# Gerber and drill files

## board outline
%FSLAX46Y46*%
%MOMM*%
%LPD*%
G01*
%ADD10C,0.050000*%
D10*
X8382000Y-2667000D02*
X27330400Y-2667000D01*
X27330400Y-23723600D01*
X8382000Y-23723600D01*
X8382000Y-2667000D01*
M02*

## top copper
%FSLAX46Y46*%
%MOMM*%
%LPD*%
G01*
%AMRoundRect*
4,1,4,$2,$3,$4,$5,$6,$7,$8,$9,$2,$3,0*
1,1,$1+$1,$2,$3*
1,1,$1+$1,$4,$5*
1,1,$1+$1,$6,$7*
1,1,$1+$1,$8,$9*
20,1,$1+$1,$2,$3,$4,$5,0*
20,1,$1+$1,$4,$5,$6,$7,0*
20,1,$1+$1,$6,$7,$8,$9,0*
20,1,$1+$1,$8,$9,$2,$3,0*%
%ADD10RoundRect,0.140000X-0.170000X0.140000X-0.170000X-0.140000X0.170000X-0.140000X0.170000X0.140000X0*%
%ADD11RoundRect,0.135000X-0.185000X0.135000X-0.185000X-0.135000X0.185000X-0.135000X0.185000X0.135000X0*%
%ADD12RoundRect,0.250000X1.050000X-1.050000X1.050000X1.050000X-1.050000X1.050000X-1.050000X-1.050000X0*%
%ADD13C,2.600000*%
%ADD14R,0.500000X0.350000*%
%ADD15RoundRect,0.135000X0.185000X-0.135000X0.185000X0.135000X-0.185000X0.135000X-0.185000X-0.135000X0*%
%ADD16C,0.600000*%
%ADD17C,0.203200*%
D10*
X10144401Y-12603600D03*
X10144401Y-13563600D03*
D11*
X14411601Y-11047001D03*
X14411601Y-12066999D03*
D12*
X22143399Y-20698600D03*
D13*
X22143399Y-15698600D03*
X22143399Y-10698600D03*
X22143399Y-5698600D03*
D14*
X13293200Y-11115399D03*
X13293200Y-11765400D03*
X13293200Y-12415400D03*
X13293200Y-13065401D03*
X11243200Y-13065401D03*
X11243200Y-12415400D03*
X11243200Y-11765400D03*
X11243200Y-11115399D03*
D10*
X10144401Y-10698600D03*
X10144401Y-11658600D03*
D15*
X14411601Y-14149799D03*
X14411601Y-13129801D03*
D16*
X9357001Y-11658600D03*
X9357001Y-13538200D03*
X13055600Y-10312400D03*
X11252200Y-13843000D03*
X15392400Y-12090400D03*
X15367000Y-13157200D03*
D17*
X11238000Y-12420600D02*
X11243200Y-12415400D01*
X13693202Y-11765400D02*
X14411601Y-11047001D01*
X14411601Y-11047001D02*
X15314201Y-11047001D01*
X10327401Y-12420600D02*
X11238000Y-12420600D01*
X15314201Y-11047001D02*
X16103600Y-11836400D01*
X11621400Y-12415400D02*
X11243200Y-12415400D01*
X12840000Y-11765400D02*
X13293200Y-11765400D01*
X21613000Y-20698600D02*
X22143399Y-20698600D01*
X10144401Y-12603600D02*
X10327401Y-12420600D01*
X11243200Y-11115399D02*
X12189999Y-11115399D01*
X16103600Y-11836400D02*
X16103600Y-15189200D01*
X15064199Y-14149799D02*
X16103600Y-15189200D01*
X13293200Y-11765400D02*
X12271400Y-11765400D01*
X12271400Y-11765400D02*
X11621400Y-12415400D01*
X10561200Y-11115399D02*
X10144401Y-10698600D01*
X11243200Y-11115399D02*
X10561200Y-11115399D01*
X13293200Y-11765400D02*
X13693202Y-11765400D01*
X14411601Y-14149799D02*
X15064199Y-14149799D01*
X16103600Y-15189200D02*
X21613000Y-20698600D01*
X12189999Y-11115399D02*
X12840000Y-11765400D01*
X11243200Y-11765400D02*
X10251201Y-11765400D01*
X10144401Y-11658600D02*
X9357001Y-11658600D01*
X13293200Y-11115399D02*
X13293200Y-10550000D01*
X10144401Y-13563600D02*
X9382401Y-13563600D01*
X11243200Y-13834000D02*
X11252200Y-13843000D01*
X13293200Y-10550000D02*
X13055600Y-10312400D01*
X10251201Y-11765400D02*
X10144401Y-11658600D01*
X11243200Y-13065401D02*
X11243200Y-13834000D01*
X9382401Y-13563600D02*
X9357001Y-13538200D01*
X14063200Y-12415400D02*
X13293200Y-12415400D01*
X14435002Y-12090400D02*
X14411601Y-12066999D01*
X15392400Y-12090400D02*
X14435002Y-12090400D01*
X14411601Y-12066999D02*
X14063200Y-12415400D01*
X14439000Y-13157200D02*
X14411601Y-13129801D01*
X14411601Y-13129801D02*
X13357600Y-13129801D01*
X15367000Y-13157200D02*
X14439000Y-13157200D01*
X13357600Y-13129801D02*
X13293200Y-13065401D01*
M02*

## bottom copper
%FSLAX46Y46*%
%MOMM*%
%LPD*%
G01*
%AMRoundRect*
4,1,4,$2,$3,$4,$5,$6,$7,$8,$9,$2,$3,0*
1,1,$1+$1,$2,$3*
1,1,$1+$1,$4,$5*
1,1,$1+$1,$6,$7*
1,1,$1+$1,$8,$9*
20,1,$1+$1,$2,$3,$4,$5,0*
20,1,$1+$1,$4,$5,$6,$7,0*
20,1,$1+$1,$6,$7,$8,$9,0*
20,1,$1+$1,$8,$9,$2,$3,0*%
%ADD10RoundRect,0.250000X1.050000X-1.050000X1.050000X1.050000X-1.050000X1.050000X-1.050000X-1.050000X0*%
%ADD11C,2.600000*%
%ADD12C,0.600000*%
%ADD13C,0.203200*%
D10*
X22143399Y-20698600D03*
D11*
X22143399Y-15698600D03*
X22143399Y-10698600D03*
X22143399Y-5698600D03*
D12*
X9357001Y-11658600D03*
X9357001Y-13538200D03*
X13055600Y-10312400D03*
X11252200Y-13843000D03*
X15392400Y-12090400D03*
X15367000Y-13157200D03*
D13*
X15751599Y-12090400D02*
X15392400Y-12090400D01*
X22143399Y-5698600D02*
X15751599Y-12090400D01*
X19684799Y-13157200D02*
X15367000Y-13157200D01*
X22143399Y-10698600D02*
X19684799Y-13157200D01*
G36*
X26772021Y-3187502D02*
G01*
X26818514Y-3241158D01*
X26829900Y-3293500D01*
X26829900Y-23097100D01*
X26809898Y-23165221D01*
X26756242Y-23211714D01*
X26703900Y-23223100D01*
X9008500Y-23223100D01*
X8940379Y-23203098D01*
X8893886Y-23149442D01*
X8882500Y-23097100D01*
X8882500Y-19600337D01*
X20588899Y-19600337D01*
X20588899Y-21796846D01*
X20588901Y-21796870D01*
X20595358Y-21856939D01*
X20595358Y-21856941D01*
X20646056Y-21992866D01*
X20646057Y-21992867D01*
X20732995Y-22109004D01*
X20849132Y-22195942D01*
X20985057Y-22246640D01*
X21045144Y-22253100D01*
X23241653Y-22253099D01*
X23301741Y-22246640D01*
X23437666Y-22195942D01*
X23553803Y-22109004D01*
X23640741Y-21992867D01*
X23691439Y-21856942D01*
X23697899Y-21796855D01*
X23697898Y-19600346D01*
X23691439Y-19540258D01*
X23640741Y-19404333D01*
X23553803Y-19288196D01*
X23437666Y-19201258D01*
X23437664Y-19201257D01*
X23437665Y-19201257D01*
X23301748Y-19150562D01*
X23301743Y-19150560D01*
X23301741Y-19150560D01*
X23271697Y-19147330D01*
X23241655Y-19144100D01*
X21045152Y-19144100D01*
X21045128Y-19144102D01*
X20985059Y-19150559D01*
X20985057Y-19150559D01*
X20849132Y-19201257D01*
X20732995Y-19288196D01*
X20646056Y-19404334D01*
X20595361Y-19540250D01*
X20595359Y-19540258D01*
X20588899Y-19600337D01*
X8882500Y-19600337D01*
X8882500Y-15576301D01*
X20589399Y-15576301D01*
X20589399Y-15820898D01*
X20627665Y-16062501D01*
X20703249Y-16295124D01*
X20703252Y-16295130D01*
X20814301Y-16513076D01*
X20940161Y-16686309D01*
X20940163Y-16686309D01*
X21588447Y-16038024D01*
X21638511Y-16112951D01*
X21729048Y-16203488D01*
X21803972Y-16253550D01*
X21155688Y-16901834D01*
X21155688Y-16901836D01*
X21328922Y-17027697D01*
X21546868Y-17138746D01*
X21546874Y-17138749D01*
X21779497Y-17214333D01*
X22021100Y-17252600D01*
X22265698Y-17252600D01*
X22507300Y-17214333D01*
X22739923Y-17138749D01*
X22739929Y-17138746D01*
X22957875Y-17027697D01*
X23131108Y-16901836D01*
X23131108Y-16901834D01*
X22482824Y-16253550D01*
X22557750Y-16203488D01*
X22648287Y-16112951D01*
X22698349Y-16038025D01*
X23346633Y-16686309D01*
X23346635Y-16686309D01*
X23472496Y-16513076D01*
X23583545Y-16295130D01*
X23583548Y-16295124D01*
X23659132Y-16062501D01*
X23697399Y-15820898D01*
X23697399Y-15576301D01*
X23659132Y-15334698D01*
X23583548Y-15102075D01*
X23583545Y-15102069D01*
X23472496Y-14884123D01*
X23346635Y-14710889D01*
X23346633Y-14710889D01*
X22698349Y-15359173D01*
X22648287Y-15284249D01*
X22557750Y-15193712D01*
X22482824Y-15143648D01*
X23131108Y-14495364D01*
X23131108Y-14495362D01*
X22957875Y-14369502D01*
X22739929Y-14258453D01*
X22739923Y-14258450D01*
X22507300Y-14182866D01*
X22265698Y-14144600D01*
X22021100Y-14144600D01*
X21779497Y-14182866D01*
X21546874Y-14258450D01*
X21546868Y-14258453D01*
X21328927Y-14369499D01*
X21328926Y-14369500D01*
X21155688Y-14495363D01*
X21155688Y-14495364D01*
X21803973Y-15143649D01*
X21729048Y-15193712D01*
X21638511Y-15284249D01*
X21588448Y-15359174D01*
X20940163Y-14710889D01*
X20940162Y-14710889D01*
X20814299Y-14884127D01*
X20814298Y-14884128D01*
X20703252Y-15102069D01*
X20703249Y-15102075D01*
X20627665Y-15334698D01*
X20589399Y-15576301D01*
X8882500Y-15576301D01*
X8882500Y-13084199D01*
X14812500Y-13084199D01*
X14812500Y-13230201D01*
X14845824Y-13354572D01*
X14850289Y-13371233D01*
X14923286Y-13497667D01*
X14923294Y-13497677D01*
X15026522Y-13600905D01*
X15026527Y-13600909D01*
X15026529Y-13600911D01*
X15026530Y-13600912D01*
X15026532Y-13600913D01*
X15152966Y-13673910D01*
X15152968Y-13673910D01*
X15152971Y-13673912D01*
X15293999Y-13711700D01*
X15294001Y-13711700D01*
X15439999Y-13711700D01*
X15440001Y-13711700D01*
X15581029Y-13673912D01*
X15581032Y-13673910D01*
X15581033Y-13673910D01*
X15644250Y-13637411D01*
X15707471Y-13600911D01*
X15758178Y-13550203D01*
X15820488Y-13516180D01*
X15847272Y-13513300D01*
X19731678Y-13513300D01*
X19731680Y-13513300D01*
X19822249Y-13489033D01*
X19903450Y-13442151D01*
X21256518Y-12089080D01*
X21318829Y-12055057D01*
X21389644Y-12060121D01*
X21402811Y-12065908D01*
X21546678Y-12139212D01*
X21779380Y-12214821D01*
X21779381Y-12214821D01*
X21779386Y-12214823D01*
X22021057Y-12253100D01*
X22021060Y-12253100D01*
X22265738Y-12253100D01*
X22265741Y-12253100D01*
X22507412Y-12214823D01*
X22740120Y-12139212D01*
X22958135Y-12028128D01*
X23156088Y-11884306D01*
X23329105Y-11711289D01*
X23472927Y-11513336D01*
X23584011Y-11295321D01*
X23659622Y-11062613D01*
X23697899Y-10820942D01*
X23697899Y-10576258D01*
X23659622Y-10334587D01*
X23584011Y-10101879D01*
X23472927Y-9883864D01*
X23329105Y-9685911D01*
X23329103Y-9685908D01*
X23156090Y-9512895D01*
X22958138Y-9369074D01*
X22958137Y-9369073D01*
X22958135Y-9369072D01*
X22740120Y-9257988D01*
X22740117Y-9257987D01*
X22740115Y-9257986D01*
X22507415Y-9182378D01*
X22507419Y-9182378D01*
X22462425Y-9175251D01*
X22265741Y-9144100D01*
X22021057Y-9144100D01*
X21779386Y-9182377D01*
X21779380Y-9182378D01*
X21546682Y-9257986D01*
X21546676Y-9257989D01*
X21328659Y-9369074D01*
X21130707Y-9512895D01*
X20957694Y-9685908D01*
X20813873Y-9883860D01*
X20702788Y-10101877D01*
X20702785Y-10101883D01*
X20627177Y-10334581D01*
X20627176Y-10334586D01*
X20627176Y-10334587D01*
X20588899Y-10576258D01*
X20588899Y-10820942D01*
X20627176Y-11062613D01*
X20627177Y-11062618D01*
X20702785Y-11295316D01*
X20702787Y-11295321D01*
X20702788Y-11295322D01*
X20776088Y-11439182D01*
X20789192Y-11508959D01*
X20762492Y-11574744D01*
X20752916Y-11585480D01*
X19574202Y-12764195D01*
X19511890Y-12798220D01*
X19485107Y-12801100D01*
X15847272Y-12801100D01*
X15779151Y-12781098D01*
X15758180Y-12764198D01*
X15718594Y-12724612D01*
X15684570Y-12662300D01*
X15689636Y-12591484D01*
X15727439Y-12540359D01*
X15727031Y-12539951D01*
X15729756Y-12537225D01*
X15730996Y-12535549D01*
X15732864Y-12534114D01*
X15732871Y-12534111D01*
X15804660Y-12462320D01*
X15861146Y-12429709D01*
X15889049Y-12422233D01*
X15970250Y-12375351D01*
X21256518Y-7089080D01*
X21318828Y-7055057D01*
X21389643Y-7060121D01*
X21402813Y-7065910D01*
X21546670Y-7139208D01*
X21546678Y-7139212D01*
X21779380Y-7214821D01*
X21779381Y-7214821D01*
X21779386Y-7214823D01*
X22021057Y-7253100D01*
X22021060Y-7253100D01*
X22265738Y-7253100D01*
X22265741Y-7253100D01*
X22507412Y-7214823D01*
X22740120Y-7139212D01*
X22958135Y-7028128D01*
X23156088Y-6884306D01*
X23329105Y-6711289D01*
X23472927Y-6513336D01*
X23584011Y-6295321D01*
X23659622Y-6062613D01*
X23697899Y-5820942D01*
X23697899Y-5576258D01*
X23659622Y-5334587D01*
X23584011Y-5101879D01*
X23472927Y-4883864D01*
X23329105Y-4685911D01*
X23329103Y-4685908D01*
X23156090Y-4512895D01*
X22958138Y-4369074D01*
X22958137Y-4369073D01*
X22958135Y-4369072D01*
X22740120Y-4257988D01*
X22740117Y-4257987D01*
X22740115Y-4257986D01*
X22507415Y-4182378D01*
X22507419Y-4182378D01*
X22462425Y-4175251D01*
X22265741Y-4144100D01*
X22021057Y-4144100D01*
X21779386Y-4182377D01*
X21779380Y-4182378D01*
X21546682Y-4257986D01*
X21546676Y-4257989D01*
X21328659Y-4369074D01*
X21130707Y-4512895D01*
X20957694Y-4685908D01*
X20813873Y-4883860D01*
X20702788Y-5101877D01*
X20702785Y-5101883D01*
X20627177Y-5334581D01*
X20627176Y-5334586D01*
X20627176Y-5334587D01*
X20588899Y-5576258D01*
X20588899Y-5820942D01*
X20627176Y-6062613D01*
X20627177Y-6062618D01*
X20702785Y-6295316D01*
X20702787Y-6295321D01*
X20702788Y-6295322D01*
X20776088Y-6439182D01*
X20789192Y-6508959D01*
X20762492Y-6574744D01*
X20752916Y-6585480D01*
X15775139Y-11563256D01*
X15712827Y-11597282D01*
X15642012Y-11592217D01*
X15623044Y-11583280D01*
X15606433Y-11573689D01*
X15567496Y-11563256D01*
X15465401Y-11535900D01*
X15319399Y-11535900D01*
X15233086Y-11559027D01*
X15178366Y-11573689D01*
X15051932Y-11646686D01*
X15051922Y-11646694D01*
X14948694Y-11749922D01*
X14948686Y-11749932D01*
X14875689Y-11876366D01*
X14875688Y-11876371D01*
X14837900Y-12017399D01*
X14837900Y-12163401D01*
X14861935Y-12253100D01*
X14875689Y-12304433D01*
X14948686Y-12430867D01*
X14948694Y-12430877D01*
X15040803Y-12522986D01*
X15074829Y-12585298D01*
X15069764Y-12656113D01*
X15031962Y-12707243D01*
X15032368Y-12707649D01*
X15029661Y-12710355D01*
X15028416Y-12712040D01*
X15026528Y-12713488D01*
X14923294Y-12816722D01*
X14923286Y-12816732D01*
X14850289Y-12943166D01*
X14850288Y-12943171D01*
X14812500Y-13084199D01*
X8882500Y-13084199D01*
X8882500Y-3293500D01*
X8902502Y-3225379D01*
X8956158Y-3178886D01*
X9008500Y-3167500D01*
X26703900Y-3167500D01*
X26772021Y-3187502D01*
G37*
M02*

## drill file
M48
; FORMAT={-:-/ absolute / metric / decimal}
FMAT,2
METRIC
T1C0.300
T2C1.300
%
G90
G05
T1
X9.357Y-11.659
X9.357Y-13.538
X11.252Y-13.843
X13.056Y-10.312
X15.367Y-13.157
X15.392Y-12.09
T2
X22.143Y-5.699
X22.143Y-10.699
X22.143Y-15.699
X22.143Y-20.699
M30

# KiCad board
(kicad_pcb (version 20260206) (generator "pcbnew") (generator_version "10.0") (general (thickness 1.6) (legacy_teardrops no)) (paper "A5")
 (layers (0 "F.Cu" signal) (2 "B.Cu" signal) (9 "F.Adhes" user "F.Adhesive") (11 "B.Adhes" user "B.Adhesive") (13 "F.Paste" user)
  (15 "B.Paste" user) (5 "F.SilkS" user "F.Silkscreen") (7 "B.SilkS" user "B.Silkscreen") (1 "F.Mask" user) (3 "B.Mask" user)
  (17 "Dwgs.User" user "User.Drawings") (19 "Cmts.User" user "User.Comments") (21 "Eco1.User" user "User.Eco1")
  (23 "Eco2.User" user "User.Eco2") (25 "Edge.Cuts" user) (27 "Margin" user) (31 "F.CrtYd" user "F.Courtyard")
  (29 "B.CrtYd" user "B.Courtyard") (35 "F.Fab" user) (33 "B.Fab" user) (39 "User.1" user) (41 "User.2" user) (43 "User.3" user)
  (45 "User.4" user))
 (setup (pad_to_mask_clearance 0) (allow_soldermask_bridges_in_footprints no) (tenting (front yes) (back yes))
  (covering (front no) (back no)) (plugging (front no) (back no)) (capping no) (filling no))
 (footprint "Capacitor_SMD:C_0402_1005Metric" (layer "F.Cu") (at 10.144401 13.0836 -90)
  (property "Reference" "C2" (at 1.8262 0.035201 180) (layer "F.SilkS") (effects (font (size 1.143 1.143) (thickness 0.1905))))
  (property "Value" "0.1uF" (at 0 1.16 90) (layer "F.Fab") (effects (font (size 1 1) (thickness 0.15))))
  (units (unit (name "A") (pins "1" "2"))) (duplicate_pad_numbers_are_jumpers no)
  (pad "1" smd roundrect (at -0.48 0 270) (size 0.56 0.62) (layers "F.Cu" "F.Mask" "F.Paste") (roundrect_rratio 0.25) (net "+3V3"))
  (pad "2" smd roundrect (at 0.48 0 270) (size 0.56 0.62) (layers "F.Cu" "F.Mask" "F.Paste") (roundrect_rratio 0.25) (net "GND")))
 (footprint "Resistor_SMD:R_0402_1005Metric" (layer "F.Cu") (at 14.411601 11.557 -90)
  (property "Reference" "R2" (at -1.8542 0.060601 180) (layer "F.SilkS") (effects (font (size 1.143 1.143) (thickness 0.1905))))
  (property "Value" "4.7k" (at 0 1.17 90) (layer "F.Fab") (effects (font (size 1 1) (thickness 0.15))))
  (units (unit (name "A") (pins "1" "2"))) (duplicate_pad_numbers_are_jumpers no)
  (pad "1" smd roundrect (at -0.509999 0 270) (size 0.54 0.64) (layers "F.Cu" "F.Mask" "F.Paste") (roundrect_rratio 0.25) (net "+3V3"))
  (pad "2" smd roundrect (at 0.509999 0 270) (size 0.54 0.64) (layers "F.Cu" "F.Mask" "F.Paste") (roundrect_rratio 0.25) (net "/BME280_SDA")))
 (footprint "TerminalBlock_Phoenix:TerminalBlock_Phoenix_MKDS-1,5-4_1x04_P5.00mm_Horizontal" (layer "F.Cu") (at 22.143399 20.6986 90)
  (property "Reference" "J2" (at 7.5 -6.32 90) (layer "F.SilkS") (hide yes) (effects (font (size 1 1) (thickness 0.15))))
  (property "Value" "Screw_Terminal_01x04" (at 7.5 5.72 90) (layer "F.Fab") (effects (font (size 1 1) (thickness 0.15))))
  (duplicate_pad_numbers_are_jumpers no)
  (pad "1" thru_hole roundrect (at 0 0 90) (size 2.6 2.6) (drill 1.3) (layers "*.Cu" "*.Mask") (remove_unused_layers no)
   (roundrect_rratio 0.096154) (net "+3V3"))
  (pad "2" thru_hole circle (at 5 0 90) (size 2.6 2.6) (drill 1.3) (layers "*.Cu" "*.Mask") (remove_unused_layers no) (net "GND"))
  (pad "3" thru_hole circle (at 10 0 90) (size 2.6 2.6) (drill 1.3) (layers "*.Cu" "*.Mask") (remove_unused_layers no) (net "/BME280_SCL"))
  (pad "4" thru_hole circle (at 15 0 90) (size 2.6 2.6) (drill 1.3) (layers "*.Cu" "*.Mask") (remove_unused_layers no) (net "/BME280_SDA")))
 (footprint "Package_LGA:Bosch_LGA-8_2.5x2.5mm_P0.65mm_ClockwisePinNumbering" (layer "F.Cu") (at 12.2682 12.0904 -90)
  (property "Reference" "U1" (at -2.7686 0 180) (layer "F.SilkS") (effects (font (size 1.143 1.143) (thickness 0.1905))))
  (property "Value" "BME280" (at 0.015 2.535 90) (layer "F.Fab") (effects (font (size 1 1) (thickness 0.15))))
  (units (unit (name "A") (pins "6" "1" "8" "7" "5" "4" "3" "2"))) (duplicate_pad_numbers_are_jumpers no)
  (pad "1" smd rect (at -0.975001 -1.025) (size 0.5 0.35) (layers "F.Cu" "F.Mask" "F.Paste") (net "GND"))
  (pad "2" smd rect (at -0.325 -1.025) (size 0.5 0.35) (layers "F.Cu" "F.Mask" "F.Paste") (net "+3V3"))
  (pad "3" smd rect (at 0.325 -1.025) (size 0.5 0.35) (layers "F.Cu" "F.Mask" "F.Paste") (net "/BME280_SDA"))
  (pad "4" smd rect (at 0.975001 -1.025) (size 0.5 0.35) (layers "F.Cu" "F.Mask" "F.Paste") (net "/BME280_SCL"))
  (pad "5" smd rect (at 0.975001 1.025) (size 0.5 0.35) (layers "F.Cu" "F.Mask" "F.Paste") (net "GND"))
  (pad "6" smd rect (at 0.325 1.025) (size 0.5 0.35) (layers "F.Cu" "F.Mask" "F.Paste") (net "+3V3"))
  (pad "7" smd rect (at -0.325 1.025) (size 0.5 0.35) (layers "F.Cu" "F.Mask" "F.Paste") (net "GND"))
  (pad "8" smd rect (at -0.975001 1.025) (size 0.5 0.35) (layers "F.Cu" "F.Mask" "F.Paste") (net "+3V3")))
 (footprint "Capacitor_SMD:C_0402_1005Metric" (layer "F.Cu") (at 10.144401 11.1786 -90)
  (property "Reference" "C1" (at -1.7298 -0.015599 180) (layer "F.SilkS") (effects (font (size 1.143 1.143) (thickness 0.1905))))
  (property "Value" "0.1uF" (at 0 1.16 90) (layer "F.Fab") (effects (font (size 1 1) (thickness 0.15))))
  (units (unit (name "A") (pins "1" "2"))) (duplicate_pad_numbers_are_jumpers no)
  (pad "1" smd roundrect (at -0.48 0 270) (size 0.56 0.62) (layers "F.Cu" "F.Mask" "F.Paste") (roundrect_rratio 0.25) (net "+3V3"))
  (pad "2" smd roundrect (at 0.48 0 270) (size 0.56 0.62) (layers "F.Cu" "F.Mask" "F.Paste") (roundrect_rratio 0.25) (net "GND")))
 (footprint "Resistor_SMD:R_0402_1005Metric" (layer "F.Cu") (at 14.411601 13.6398 90)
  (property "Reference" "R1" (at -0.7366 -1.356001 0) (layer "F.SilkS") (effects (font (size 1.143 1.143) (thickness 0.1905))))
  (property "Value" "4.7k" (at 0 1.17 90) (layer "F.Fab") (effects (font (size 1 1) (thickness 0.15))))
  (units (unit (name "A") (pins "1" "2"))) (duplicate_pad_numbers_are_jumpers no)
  (pad "1" smd roundrect (at -0.509999 0 90) (size 0.54 0.64) (layers "F.Cu" "F.Mask" "F.Paste") (roundrect_rratio 0.25) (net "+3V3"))
  (pad "2" smd roundrect (at 0.509999 0 90) (size 0.54 0.64) (layers "F.Cu" "F.Mask" "F.Paste") (roundrect_rratio 0.25) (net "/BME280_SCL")))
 (gr_rect (start 8.382 2.667) (end 27.3304 23.7236) (stroke (width 0.05) (type default)) (fill no) (layer "Edge.Cuts"))
 (segment (start 11.238 12.4206) (end 11.2432 12.4154) (width 0.2032) (layer "F.Cu") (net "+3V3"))
 (segment (start 13.693202 11.7654) (end 14.411601 11.047001) (width 0.2032) (layer "F.Cu") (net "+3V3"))
 (segment (start 14.411601 11.047001) (end 15.314201 11.047001) (width 0.2032) (layer "F.Cu") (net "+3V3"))
 (segment (start 10.327401 12.4206) (end 11.238 12.4206) (width 0.2032) (layer "F.Cu") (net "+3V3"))
 (segment (start 15.314201 11.047001) (end 16.1036 11.8364) (width 0.2032) (layer "F.Cu") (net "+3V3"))
 (segment (start 11.6214 12.4154) (end 11.2432 12.4154) (width 0.2032) (layer "F.Cu") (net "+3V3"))
 (segment (start 12.84 11.7654) (end 13.2932 11.7654) (width 0.2032) (layer "F.Cu") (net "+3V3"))
 (segment (start 21.613 20.6986) (end 22.143399 20.6986) (width 0.2032) (layer "F.Cu") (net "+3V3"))
 (segment (start 10.144401 12.6036) (end 10.327401 12.4206) (width 0.2032) (layer "F.Cu") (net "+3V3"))
 (segment (start 11.2432 11.115399) (end 12.189999 11.115399) (width 0.2032) (layer "F.Cu") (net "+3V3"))
 (segment (start 16.1036 11.8364) (end 16.1036 15.1892) (width 0.2032) (layer "F.Cu") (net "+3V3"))
 (segment (start 15.064199 14.149799) (end 16.1036 15.1892) (width 0.2032) (layer "F.Cu") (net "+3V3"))
 (segment (start 13.2932 11.7654) (end 12.2714 11.7654) (width 0.2032) (layer "F.Cu") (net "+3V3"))
 (segment (start 12.2714 11.7654) (end 11.6214 12.4154) (width 0.2032) (layer "F.Cu") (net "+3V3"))
 (segment (start 10.5612 11.115399) (end 10.144401 10.6986) (width 0.2032) (layer "F.Cu") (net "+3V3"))
 (segment (start 11.2432 11.115399) (end 10.5612 11.115399) (width 0.2032) (layer "F.Cu") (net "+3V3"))
 (segment (start 13.2932 11.7654) (end 13.693202 11.7654) (width 0.2032) (layer "F.Cu") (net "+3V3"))
 (segment (start 14.411601 14.149799) (end 15.064199 14.149799) (width 0.2032) (layer "F.Cu") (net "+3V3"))
 (segment (start 16.1036 15.1892) (end 21.613 20.6986) (width 0.2032) (layer "F.Cu") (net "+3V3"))
 (segment (start 12.189999 11.115399) (end 12.84 11.7654) (width 0.2032) (layer "F.Cu") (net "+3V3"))
 (segment (start 11.2432 11.7654) (end 10.251201 11.7654) (width 0.2032) (layer "F.Cu") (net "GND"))
 (segment (start 10.144401 11.6586) (end 9.357001 11.6586) (width 0.2032) (layer "F.Cu") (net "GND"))
 (segment (start 13.2932 11.115399) (end 13.2932 10.55) (width 0.2032) (layer "F.Cu") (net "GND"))
 (segment (start 10.144401 13.5636) (end 9.382401 13.5636) (width 0.2032) (layer "F.Cu") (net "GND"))
 (segment (start 11.2432 13.834) (end 11.2522 13.843) (width 0.2032) (layer "F.Cu") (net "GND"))
 (segment (start 13.2932 10.55) (end 13.0556 10.3124) (width 0.2032) (layer "F.Cu") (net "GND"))
 (segment (start 10.251201 11.7654) (end 10.144401 11.6586) (width 0.2032) (layer "F.Cu") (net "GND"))
 (segment (start 11.2432 13.065401) (end 11.2432 13.834) (width 0.2032) (layer "F.Cu") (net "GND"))
 (segment (start 9.382401 13.5636) (end 9.357001 13.5382) (width 0.2032) (layer "F.Cu") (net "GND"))
 (via (at 9.357001 11.6586) (size 0.6) (drill 0.3) (layers "F.Cu" "B.Cu") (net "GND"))
 (via (at 9.357001 13.5382) (size 0.6) (drill 0.3) (layers "F.Cu" "B.Cu") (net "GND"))
 (via (at 13.0556 10.3124) (size 0.6) (drill 0.3) (layers "F.Cu" "B.Cu") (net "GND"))
 (via (at 11.2522 13.843) (size 0.6) (drill 0.3) (layers "F.Cu" "B.Cu") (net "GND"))
 (segment (start 14.0632 12.4154) (end 13.2932 12.4154) (width 0.2032) (layer "F.Cu") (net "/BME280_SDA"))
 (segment (start 14.435002 12.0904) (end 14.411601 12.066999) (width 0.2032) (layer "F.Cu") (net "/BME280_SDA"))
 (segment (start 15.3924 12.0904) (end 14.435002 12.0904) (width 0.2032) (layer "F.Cu") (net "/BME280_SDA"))
 (segment (start 14.411601 12.066999) (end 14.0632 12.4154) (width 0.2032) (layer "F.Cu") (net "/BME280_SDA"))
 (via (at 15.3924 12.0904) (size 0.6) (drill 0.3) (layers "F.Cu" "B.Cu") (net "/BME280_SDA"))
 (segment (start 15.751599 12.0904) (end 15.3924 12.0904) (width 0.2032) (layer "B.Cu") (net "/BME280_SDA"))
 (segment (start 22.143399 5.6986) (end 15.751599 12.0904) (width 0.2032) (layer "B.Cu") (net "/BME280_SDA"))
 (segment (start 14.439 13.1572) (end 14.411601 13.129801) (width 0.2032) (layer "F.Cu") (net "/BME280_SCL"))
 (segment (start 14.411601 13.129801) (end 13.3576 13.129801) (width 0.2032) (layer "F.Cu") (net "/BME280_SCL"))
 (segment (start 15.367 13.1572) (end 14.439 13.1572) (width 0.2032) (layer "F.Cu") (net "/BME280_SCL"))
 (segment (start 13.3576 13.129801) (end 13.2932 13.065401) (width 0.2032) (layer "F.Cu") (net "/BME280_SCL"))
 (via (at 15.367 13.1572) (size 0.6) (drill 0.3) (layers "F.Cu" "B.Cu") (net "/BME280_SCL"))
 (segment (start 19.684799 13.1572) (end 15.367 13.1572) (width 0.2032) (layer "B.Cu") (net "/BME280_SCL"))
 (segment (start 22.143399 10.6986) (end 19.684799 13.1572) (width 0.2032) (layer "B.Cu") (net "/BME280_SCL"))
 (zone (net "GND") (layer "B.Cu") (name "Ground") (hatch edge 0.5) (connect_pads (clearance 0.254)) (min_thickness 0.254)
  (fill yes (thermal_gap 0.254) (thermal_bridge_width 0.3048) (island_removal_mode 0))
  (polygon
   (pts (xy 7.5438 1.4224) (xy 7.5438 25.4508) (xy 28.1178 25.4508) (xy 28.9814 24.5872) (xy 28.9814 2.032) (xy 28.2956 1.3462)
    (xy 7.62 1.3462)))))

